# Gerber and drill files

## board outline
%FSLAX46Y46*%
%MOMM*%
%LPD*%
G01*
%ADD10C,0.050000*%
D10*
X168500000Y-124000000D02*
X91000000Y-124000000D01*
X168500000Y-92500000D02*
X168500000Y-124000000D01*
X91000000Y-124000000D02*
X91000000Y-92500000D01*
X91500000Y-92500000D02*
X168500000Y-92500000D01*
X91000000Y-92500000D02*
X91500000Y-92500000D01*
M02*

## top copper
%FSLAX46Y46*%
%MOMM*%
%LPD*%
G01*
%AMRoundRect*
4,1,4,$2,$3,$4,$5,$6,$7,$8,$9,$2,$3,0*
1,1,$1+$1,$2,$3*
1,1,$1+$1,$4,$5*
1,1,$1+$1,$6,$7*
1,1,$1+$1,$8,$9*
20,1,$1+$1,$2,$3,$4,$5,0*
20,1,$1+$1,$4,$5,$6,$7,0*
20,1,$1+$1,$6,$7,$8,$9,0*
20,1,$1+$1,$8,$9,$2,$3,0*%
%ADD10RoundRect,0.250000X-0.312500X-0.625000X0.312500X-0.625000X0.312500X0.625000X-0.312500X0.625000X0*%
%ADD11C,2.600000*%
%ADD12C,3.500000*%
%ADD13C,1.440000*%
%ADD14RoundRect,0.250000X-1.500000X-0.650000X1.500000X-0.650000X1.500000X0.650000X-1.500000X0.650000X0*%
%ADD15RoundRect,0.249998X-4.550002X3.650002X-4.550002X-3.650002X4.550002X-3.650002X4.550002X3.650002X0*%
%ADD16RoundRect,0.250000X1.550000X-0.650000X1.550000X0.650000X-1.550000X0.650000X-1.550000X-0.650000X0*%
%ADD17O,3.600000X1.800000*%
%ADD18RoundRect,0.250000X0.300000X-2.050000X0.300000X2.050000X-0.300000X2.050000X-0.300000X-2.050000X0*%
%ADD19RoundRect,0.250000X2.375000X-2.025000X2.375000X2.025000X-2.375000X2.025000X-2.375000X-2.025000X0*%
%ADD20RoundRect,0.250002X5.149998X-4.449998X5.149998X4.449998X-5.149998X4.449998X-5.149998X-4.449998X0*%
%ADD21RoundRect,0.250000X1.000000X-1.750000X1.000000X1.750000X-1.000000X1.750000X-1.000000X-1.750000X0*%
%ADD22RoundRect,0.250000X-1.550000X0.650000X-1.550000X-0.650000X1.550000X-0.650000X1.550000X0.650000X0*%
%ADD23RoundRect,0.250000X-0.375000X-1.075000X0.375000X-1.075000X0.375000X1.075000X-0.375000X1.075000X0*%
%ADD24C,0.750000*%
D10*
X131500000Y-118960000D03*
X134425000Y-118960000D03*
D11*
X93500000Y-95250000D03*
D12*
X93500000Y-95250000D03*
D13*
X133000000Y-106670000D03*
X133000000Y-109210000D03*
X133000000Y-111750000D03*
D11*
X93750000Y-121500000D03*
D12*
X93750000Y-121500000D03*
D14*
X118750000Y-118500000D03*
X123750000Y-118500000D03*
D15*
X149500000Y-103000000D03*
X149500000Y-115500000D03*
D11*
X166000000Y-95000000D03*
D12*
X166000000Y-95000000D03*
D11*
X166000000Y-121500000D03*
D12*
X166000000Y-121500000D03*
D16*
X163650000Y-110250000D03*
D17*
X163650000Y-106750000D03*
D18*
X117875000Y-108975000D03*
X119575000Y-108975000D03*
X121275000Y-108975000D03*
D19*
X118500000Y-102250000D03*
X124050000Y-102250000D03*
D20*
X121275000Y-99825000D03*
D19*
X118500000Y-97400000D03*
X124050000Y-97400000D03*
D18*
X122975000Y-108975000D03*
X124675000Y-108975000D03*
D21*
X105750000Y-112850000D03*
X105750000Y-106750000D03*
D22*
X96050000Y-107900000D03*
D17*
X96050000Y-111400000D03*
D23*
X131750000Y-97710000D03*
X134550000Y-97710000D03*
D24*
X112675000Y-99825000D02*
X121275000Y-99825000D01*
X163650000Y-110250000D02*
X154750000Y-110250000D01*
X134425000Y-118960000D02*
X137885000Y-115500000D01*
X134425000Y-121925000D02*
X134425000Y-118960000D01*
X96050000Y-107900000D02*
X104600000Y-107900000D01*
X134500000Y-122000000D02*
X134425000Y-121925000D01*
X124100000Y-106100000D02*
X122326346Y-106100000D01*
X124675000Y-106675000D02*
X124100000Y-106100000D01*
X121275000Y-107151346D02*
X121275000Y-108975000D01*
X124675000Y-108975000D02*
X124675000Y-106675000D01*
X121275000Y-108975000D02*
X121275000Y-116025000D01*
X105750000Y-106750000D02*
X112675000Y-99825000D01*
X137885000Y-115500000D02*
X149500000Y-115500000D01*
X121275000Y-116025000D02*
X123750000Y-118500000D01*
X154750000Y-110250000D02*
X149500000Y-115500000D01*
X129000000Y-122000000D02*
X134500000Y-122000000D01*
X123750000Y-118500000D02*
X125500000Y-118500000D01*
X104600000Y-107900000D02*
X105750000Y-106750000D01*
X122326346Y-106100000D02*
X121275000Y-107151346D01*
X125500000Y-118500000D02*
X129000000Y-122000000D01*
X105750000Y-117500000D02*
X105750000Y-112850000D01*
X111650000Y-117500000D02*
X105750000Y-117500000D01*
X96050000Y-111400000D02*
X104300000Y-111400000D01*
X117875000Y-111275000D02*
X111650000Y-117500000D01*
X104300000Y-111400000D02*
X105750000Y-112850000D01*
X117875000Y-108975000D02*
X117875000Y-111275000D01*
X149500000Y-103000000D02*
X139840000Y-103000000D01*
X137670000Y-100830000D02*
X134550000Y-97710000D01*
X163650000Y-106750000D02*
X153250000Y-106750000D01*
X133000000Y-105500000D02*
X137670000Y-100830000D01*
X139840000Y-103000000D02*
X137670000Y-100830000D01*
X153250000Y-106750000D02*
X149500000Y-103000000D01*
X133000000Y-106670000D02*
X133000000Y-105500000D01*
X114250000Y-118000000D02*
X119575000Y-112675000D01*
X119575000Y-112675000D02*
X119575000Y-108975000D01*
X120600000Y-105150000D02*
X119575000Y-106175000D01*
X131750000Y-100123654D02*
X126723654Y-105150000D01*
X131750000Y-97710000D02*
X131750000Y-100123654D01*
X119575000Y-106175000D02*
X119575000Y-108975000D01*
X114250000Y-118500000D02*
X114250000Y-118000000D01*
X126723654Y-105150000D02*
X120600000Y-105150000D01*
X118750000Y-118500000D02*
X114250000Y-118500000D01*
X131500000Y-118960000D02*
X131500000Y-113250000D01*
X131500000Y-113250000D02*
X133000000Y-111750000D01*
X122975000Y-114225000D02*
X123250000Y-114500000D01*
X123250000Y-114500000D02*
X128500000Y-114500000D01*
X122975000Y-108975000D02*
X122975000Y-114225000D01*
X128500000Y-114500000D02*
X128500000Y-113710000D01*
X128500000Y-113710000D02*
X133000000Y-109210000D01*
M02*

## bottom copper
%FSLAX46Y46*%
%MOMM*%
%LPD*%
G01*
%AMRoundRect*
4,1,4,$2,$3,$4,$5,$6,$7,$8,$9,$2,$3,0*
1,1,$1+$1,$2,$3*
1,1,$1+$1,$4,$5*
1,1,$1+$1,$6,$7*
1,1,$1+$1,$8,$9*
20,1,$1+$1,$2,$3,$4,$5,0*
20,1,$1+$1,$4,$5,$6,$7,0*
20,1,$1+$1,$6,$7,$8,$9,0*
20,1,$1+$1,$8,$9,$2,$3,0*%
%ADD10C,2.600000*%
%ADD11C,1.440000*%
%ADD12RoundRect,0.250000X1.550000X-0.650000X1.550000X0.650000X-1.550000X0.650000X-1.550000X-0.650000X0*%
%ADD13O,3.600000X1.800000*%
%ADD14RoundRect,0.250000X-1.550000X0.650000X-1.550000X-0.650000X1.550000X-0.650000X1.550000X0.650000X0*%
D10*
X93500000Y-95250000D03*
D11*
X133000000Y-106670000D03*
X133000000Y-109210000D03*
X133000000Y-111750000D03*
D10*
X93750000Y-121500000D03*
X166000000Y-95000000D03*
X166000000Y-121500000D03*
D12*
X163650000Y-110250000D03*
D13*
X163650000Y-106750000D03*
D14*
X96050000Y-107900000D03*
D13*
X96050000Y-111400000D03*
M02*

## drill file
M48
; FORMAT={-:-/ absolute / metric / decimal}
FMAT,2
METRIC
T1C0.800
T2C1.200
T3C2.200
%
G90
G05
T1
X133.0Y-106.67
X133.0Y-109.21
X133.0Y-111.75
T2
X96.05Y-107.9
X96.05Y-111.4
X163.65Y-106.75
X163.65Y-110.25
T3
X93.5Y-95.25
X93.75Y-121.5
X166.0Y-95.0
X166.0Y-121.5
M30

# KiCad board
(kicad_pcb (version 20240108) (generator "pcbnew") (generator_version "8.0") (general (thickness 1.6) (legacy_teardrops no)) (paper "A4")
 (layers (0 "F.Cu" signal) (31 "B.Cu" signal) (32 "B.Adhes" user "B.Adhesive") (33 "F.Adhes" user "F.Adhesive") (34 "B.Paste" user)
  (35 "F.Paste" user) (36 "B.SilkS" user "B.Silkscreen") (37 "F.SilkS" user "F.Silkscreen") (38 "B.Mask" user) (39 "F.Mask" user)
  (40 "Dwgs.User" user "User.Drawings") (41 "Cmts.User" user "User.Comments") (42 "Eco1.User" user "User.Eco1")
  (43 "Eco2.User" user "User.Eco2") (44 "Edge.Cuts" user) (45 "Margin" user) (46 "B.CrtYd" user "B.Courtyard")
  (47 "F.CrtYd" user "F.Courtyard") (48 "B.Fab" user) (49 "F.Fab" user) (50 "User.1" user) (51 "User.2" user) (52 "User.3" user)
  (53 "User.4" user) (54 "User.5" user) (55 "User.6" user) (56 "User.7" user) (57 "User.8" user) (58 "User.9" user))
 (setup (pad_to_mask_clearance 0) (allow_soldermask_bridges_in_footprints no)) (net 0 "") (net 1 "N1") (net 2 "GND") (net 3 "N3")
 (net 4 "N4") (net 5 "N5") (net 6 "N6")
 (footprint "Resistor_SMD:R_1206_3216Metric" (layer "F.Cu") (at 132.9625 118.96)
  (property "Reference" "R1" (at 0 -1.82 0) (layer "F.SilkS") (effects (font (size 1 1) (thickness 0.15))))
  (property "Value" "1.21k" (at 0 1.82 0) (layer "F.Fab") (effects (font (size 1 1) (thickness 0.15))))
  (pad "1" smd roundrect (at -1.4625 0) (size 1.125 1.75) (layers "F.Cu" "F.Paste" "F.Mask") (roundrect_rratio 0.222222) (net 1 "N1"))
  (pad "2" smd roundrect (at 1.4625 0) (size 1.125 1.75) (layers "F.Cu" "F.Paste" "F.Mask") (roundrect_rratio 0.222222) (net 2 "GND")))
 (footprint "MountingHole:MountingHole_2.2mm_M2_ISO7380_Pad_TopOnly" (layer "F.Cu") (at 93.5 95.25)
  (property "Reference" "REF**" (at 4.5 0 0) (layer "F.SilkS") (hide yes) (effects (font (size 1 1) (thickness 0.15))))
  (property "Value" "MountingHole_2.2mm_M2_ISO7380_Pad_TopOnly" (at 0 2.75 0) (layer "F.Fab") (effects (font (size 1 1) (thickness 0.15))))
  (pad "1" thru_hole circle (at 0 0) (size 2.6 2.6) (drill 2.2) (layers "*.Cu" "*.Mask") (remove_unused_layers no))
  (pad "1" connect circle (at 0 0) (size 3.5 3.5) (layers "F.Cu" "F.Mask")))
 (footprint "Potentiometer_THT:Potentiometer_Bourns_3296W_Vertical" (layer "F.Cu") (at 133 106.67 90)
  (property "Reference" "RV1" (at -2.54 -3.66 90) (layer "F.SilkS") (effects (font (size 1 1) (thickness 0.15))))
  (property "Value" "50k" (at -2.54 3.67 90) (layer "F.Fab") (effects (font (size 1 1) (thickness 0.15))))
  (pad "1" thru_hole circle (at 0 0 90) (size 1.44 1.44) (drill 0.8) (layers "*.Cu" "*.Mask") (remove_unused_layers no) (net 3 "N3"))
  (pad "2" thru_hole circle (at -2.54 0 90) (size 1.44 1.44) (drill 0.8) (layers "*.Cu" "*.Mask") (remove_unused_layers no) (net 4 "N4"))
  (pad "3" thru_hole circle (at -5.08 0 90) (size 1.44 1.44) (drill 0.8) (layers "*.Cu" "*.Mask") (remove_unused_layers no) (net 1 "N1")))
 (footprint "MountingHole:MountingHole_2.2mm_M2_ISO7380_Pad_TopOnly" (layer "F.Cu") (at 93.75 121.5)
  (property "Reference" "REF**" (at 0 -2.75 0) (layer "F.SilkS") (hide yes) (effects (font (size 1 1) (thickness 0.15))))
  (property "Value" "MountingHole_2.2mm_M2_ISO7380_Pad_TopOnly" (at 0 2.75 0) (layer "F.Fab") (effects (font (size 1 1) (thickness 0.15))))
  (pad "1" thru_hole circle (at 0 0) (size 2.6 2.6) (drill 2.2) (layers "*.Cu" "*.Mask") (remove_unused_layers no))
  (pad "1" connect circle (at 0 0) (size 3.5 3.5) (layers "F.Cu" "F.Mask")))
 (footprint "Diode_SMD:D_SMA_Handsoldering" (layer "F.Cu") (at 121.25 118.5)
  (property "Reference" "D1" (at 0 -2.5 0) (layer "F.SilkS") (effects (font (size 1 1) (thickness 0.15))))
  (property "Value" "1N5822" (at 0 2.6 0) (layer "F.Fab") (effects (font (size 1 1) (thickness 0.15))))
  (pad "1" smd roundrect (at -2.5 0) (size 3.5 1.8) (layers "F.Cu" "F.Paste" "F.Mask") (roundrect_rratio 0.1388888889) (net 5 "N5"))
  (pad "2" smd roundrect (at 2.5 0) (size 3.5 1.8) (layers "F.Cu" "F.Paste" "F.Mask") (roundrect_rratio 0.1388888889) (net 2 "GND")))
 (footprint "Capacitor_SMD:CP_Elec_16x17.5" (layer "F.Cu") (at 149.5 109.25 -90)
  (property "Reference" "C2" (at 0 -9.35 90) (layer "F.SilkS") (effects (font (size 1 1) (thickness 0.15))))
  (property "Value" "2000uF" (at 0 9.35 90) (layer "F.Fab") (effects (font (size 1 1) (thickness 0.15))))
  (pad "1" smd roundrect (at -6.25 0 270) (size 7.8 9.6) (layers "F.Cu" "F.Paste" "F.Mask") (roundrect_rratio 0.032051) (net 3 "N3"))
  (pad "2" smd roundrect (at 6.25 0 270) (size 7.8 9.6) (layers "F.Cu" "F.Paste" "F.Mask") (roundrect_rratio 0.032051) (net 2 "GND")))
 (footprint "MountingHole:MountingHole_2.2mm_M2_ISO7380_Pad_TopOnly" (layer "F.Cu") (at 166 95)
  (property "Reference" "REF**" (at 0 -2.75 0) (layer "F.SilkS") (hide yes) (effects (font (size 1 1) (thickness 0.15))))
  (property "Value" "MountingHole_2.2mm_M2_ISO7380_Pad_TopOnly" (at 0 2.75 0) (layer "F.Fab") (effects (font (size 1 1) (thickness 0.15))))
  (pad "1" thru_hole circle (at 0 0) (size 2.6 2.6) (drill 2.2) (layers "*.Cu" "*.Mask") (remove_unused_layers no))
  (pad "1" connect circle (at 0 0) (size 3.5 3.5) (layers "F.Cu" "F.Mask")))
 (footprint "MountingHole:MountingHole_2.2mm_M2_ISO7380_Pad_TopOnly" (layer "F.Cu") (at 166 121.5)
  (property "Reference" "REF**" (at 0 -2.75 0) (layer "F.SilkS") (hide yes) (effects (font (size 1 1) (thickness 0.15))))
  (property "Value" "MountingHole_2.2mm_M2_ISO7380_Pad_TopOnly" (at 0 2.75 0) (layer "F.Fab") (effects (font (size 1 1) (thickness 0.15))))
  (pad "1" thru_hole circle (at 0 0) (size 2.6 2.6) (drill 2.2) (layers "*.Cu" "*.Mask") (remove_unused_layers no))
  (pad "1" connect circle (at 0 0) (size 3.5 3.5) (layers "F.Cu" "F.Mask")))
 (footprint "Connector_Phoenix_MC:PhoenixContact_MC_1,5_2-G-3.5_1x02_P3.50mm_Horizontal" (layer "F.Cu") (at 163.65 110.25 90)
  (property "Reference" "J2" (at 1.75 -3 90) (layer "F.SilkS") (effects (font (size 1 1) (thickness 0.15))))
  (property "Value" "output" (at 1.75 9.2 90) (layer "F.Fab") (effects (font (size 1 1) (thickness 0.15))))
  (pad "1" thru_hole roundrect (at 0 0 90) (size 1.8 3.6) (drill 1.2) (layers "*.Cu" "*.Mask") (remove_unused_layers no)
   (roundrect_rratio 0.138889) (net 2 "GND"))
  (pad "2" thru_hole oval (at 3.5 0 90) (size 1.8 3.6) (drill 1.2) (layers "*.Cu" "*.Mask") (remove_unused_layers no) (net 3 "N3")))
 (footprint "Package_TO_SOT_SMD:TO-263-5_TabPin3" (layer "F.Cu") (at 121.275 101.325 90)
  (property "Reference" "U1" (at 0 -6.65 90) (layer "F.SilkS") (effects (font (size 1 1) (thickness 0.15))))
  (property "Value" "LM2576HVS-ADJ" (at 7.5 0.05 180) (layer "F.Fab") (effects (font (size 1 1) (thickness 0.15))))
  (pad "1" smd roundrect (at -7.65 -3.4 90) (size 4.6 1.1) (layers "F.Cu" "F.Paste" "F.Mask") (roundrect_rratio 0.227273) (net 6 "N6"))
  (pad "2" smd roundrect (at -7.65 -1.7 90) (size 4.6 1.1) (layers "F.Cu" "F.Paste" "F.Mask") (roundrect_rratio 0.227273) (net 5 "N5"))
  (pad "3" smd roundrect (at -7.65 0 90) (size 4.6 1.1) (layers "F.Cu" "F.Paste" "F.Mask") (roundrect_rratio 0.227273) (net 2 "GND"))
  (pad "3" smd roundrect (at -0.925 -2.775 90) (size 4.55 5.25) (layers "F.Cu" "F.Paste") (roundrect_rratio 0.054945) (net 2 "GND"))
  (pad "3" smd roundrect (at -0.925 2.775 90) (size 4.55 5.25) (layers "F.Cu" "F.Paste") (roundrect_rratio 0.054945) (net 2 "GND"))
  (pad "3" smd roundrect (at 1.5 0 90) (size 9.4 10.8) (layers "F.Cu" "F.Mask") (roundrect_rratio 0.026596) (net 2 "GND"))
  (pad "3" smd roundrect (at 3.925 -2.775 90) (size 4.55 5.25) (layers "F.Cu" "F.Paste") (roundrect_rratio 0.054945) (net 2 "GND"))
  (pad "3" smd roundrect (at 3.925 2.775 90) (size 4.55 5.25) (layers "F.Cu" "F.Paste") (roundrect_rratio 0.054945) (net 2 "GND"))
  (pad "4" smd roundrect (at -7.65 1.7 90) (size 4.6 1.1) (layers "F.Cu" "F.Paste" "F.Mask") (roundrect_rratio 0.227273) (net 4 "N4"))
  (pad "5" smd roundrect (at -7.65 3.4 90) (size 4.6 1.1) (layers "F.Cu" "F.Paste" "F.Mask") (roundrect_rratio 0.227273) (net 2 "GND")))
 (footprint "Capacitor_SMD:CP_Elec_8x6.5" (layer "F.Cu") (at 105.75 109.8 90)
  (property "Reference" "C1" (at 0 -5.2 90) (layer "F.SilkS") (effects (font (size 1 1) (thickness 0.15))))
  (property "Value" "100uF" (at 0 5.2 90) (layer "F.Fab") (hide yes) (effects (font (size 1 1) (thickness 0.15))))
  (pad "1" smd roundrect (at -3.05 0 90) (size 4 2.5) (layers "F.Cu" "F.Paste" "F.Mask") (roundrect_rratio 0.1) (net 6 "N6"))
  (pad "2" smd roundrect (at 3.05 0 90) (size 4 2.5) (layers "F.Cu" "F.Paste" "F.Mask") (roundrect_rratio 0.1) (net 2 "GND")))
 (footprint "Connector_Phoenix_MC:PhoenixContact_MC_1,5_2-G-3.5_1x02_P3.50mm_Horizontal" (layer "F.Cu") (at 96.05 107.9 -90)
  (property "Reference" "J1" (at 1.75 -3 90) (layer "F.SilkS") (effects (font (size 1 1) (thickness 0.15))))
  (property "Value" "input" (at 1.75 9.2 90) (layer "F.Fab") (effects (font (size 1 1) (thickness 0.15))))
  (pad "1" thru_hole roundrect (at 0 0 270) (size 1.8 3.6) (drill 1.2) (layers "*.Cu" "*.Mask") (remove_unused_layers no)
   (roundrect_rratio 0.138889) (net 2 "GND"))
  (pad "2" thru_hole oval (at 3.5 0 270) (size 1.8 3.6) (drill 1.2) (layers "*.Cu" "*.Mask") (remove_unused_layers no) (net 6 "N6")))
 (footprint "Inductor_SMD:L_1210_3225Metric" (layer "F.Cu") (at 133.15 97.71)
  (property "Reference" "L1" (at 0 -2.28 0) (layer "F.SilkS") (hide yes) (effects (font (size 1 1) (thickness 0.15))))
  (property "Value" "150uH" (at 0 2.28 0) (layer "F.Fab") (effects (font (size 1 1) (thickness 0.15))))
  (pad "1" smd roundrect (at -1.4 0) (size 1.25 2.65) (layers "F.Cu" "F.Paste" "F.Mask") (roundrect_rratio 0.2) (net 5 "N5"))
  (pad "2" smd roundrect (at 1.4 0) (size 1.25 2.65) (layers "F.Cu" "F.Paste" "F.Mask") (roundrect_rratio 0.2) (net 3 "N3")))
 (gr_line (start 168.5 124) (end 91 124) (stroke (width 0.05) (type default)) (layer "Edge.Cuts"))
 (gr_line (start 168.5 92.5) (end 168.5 124) (stroke (width 0.05) (type default)) (layer "Edge.Cuts"))
 (gr_line (start 91 124) (end 91 92.5) (stroke (width 0.05) (type default)) (layer "Edge.Cuts"))
 (gr_line (start 91.5 92.5) (end 168.5 92.5) (stroke (width 0.05) (type default)) (layer "Edge.Cuts"))
 (gr_line (start 91 92.5) (end 91.5 92.5) (stroke (width 0.05) (type default)) (layer "Edge.Cuts"))
 (segment (start 112.675 99.825) (end 121.275 99.825) (width 0.75) (layer "F.Cu") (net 2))
 (segment (start 163.65 110.25) (end 154.75 110.25) (width 0.75) (layer "F.Cu") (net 2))
 (segment (start 134.425 118.96) (end 137.885 115.5) (width 0.75) (layer "F.Cu") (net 2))
 (segment (start 134.425 121.925) (end 134.425 118.96) (width 0.75) (layer "F.Cu") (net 2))
 (segment (start 96.05 107.9) (end 104.6 107.9) (width 0.75) (layer "F.Cu") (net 2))
 (segment (start 134.5 122) (end 134.425 121.925) (width 0.75) (layer "F.Cu") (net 2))
 (segment (start 124.1 106.1) (end 122.326346 106.1) (width 0.75) (layer "F.Cu") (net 2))
 (segment (start 124.675 106.675) (end 124.1 106.1) (width 0.75) (layer "F.Cu") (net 2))
 (segment (start 121.275 107.151346) (end 121.275 108.975) (width 0.75) (layer "F.Cu") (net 2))
 (segment (start 124.675 108.975) (end 124.675 106.675) (width 0.75) (layer "F.Cu") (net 2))
 (segment (start 121.275 108.975) (end 121.275 116.025) (width 0.75) (layer "F.Cu") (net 2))
 (segment (start 105.75 106.75) (end 112.675 99.825) (width 0.75) (layer "F.Cu") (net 2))
 (segment (start 137.885 115.5) (end 149.5 115.5) (width 0.75) (layer "F.Cu") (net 2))
 (segment (start 121.275 116.025) (end 123.75 118.5) (width 0.75) (layer "F.Cu") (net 2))
 (segment (start 154.75 110.25) (end 149.5 115.5) (width 0.75) (layer "F.Cu") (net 2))
 (segment (start 129 122) (end 134.5 122) (width 0.75) (layer "F.Cu") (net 2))
 (segment (start 123.75 118.5) (end 125.5 118.5) (width 0.75) (layer "F.Cu") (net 2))
 (segment (start 104.6 107.9) (end 105.75 106.75) (width 0.75) (layer "F.Cu") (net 2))
 (segment (start 122.326346 106.1) (end 121.275 107.151346) (width 0.75) (layer "F.Cu") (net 2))
 (segment (start 125.5 118.5) (end 129 122) (width 0.75) (layer "F.Cu") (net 2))
 (segment (start 105.75 117.5) (end 105.75 112.85) (width 0.75) (layer "F.Cu") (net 6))
 (segment (start 111.65 117.5) (end 105.75 117.5) (width 0.75) (layer "F.Cu") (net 6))
 (segment (start 96.05 111.4) (end 104.3 111.4) (width 0.75) (layer "F.Cu") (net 6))
 (segment (start 117.875 111.275) (end 111.65 117.5) (width 0.75) (layer "F.Cu") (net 6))
 (segment (start 104.3 111.4) (end 105.75 112.85) (width 0.75) (layer "F.Cu") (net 6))
 (segment (start 117.875 108.975) (end 117.875 111.275) (width 0.75) (layer "F.Cu") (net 6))
 (segment (start 149.5 103) (end 139.84 103) (width 0.75) (layer "F.Cu") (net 3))
 (segment (start 137.67 100.83) (end 134.55 97.71) (width 0.75) (layer "F.Cu") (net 3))
 (segment (start 163.65 106.75) (end 153.25 106.75) (width 0.75) (layer "F.Cu") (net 3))
 (segment (start 133 105.5) (end 137.67 100.83) (width 0.75) (layer "F.Cu") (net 3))
 (segment (start 139.84 103) (end 137.67 100.83) (width 0.75) (layer "F.Cu") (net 3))
 (segment (start 153.25 106.75) (end 149.5 103) (width 0.75) (layer "F.Cu") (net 3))
 (segment (start 133 106.67) (end 133 105.5) (width 0.75) (layer "F.Cu") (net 3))
 (segment (start 114.25 118) (end 119.575 112.675) (width 0.75) (layer "F.Cu") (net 5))
 (segment (start 119.575 112.675) (end 119.575 108.975) (width 0.75) (layer "F.Cu") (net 5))
 (segment (start 120.6 105.15) (end 119.575 106.175) (width 0.75) (layer "F.Cu") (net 5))
 (segment (start 131.75 100.123654) (end 126.723654 105.15) (width 0.75) (layer "F.Cu") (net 5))
 (segment (start 131.75 97.71) (end 131.75 100.123654) (width 0.75) (layer "F.Cu") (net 5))
 (segment (start 119.575 106.175) (end 119.575 108.975) (width 0.75) (layer "F.Cu") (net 5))
 (segment (start 114.25 118.5) (end 114.25 118) (width 0.75) (layer "F.Cu") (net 5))
 (segment (start 126.723654 105.15) (end 120.6 105.15) (width 0.75) (layer "F.Cu") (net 5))
 (segment (start 118.75 118.5) (end 114.25 118.5) (width 0.75) (layer "F.Cu") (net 5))
 (segment (start 131.5 118.96) (end 131.5 113.25) (width 0.75) (layer "F.Cu") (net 1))
 (segment (start 131.5 113.25) (end 133 111.75) (width 0.75) (layer "F.Cu") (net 1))
 (segment (start 122.975 114.225) (end 123.25 114.5) (width 0.75) (layer "F.Cu") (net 4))
 (segment (start 123.25 114.5) (end 128.5 114.5) (width 0.75) (layer "F.Cu") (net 4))
 (segment (start 122.975 108.975) (end 122.975 114.225) (width 0.75) (layer "F.Cu") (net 4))
 (segment (start 128.5 114.5) (end 128.5 113.71) (width 0.75) (layer "F.Cu") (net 4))
 (segment (start 128.5 113.71) (end 133 109.21) (width 0.75) (layer "F.Cu") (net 4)))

